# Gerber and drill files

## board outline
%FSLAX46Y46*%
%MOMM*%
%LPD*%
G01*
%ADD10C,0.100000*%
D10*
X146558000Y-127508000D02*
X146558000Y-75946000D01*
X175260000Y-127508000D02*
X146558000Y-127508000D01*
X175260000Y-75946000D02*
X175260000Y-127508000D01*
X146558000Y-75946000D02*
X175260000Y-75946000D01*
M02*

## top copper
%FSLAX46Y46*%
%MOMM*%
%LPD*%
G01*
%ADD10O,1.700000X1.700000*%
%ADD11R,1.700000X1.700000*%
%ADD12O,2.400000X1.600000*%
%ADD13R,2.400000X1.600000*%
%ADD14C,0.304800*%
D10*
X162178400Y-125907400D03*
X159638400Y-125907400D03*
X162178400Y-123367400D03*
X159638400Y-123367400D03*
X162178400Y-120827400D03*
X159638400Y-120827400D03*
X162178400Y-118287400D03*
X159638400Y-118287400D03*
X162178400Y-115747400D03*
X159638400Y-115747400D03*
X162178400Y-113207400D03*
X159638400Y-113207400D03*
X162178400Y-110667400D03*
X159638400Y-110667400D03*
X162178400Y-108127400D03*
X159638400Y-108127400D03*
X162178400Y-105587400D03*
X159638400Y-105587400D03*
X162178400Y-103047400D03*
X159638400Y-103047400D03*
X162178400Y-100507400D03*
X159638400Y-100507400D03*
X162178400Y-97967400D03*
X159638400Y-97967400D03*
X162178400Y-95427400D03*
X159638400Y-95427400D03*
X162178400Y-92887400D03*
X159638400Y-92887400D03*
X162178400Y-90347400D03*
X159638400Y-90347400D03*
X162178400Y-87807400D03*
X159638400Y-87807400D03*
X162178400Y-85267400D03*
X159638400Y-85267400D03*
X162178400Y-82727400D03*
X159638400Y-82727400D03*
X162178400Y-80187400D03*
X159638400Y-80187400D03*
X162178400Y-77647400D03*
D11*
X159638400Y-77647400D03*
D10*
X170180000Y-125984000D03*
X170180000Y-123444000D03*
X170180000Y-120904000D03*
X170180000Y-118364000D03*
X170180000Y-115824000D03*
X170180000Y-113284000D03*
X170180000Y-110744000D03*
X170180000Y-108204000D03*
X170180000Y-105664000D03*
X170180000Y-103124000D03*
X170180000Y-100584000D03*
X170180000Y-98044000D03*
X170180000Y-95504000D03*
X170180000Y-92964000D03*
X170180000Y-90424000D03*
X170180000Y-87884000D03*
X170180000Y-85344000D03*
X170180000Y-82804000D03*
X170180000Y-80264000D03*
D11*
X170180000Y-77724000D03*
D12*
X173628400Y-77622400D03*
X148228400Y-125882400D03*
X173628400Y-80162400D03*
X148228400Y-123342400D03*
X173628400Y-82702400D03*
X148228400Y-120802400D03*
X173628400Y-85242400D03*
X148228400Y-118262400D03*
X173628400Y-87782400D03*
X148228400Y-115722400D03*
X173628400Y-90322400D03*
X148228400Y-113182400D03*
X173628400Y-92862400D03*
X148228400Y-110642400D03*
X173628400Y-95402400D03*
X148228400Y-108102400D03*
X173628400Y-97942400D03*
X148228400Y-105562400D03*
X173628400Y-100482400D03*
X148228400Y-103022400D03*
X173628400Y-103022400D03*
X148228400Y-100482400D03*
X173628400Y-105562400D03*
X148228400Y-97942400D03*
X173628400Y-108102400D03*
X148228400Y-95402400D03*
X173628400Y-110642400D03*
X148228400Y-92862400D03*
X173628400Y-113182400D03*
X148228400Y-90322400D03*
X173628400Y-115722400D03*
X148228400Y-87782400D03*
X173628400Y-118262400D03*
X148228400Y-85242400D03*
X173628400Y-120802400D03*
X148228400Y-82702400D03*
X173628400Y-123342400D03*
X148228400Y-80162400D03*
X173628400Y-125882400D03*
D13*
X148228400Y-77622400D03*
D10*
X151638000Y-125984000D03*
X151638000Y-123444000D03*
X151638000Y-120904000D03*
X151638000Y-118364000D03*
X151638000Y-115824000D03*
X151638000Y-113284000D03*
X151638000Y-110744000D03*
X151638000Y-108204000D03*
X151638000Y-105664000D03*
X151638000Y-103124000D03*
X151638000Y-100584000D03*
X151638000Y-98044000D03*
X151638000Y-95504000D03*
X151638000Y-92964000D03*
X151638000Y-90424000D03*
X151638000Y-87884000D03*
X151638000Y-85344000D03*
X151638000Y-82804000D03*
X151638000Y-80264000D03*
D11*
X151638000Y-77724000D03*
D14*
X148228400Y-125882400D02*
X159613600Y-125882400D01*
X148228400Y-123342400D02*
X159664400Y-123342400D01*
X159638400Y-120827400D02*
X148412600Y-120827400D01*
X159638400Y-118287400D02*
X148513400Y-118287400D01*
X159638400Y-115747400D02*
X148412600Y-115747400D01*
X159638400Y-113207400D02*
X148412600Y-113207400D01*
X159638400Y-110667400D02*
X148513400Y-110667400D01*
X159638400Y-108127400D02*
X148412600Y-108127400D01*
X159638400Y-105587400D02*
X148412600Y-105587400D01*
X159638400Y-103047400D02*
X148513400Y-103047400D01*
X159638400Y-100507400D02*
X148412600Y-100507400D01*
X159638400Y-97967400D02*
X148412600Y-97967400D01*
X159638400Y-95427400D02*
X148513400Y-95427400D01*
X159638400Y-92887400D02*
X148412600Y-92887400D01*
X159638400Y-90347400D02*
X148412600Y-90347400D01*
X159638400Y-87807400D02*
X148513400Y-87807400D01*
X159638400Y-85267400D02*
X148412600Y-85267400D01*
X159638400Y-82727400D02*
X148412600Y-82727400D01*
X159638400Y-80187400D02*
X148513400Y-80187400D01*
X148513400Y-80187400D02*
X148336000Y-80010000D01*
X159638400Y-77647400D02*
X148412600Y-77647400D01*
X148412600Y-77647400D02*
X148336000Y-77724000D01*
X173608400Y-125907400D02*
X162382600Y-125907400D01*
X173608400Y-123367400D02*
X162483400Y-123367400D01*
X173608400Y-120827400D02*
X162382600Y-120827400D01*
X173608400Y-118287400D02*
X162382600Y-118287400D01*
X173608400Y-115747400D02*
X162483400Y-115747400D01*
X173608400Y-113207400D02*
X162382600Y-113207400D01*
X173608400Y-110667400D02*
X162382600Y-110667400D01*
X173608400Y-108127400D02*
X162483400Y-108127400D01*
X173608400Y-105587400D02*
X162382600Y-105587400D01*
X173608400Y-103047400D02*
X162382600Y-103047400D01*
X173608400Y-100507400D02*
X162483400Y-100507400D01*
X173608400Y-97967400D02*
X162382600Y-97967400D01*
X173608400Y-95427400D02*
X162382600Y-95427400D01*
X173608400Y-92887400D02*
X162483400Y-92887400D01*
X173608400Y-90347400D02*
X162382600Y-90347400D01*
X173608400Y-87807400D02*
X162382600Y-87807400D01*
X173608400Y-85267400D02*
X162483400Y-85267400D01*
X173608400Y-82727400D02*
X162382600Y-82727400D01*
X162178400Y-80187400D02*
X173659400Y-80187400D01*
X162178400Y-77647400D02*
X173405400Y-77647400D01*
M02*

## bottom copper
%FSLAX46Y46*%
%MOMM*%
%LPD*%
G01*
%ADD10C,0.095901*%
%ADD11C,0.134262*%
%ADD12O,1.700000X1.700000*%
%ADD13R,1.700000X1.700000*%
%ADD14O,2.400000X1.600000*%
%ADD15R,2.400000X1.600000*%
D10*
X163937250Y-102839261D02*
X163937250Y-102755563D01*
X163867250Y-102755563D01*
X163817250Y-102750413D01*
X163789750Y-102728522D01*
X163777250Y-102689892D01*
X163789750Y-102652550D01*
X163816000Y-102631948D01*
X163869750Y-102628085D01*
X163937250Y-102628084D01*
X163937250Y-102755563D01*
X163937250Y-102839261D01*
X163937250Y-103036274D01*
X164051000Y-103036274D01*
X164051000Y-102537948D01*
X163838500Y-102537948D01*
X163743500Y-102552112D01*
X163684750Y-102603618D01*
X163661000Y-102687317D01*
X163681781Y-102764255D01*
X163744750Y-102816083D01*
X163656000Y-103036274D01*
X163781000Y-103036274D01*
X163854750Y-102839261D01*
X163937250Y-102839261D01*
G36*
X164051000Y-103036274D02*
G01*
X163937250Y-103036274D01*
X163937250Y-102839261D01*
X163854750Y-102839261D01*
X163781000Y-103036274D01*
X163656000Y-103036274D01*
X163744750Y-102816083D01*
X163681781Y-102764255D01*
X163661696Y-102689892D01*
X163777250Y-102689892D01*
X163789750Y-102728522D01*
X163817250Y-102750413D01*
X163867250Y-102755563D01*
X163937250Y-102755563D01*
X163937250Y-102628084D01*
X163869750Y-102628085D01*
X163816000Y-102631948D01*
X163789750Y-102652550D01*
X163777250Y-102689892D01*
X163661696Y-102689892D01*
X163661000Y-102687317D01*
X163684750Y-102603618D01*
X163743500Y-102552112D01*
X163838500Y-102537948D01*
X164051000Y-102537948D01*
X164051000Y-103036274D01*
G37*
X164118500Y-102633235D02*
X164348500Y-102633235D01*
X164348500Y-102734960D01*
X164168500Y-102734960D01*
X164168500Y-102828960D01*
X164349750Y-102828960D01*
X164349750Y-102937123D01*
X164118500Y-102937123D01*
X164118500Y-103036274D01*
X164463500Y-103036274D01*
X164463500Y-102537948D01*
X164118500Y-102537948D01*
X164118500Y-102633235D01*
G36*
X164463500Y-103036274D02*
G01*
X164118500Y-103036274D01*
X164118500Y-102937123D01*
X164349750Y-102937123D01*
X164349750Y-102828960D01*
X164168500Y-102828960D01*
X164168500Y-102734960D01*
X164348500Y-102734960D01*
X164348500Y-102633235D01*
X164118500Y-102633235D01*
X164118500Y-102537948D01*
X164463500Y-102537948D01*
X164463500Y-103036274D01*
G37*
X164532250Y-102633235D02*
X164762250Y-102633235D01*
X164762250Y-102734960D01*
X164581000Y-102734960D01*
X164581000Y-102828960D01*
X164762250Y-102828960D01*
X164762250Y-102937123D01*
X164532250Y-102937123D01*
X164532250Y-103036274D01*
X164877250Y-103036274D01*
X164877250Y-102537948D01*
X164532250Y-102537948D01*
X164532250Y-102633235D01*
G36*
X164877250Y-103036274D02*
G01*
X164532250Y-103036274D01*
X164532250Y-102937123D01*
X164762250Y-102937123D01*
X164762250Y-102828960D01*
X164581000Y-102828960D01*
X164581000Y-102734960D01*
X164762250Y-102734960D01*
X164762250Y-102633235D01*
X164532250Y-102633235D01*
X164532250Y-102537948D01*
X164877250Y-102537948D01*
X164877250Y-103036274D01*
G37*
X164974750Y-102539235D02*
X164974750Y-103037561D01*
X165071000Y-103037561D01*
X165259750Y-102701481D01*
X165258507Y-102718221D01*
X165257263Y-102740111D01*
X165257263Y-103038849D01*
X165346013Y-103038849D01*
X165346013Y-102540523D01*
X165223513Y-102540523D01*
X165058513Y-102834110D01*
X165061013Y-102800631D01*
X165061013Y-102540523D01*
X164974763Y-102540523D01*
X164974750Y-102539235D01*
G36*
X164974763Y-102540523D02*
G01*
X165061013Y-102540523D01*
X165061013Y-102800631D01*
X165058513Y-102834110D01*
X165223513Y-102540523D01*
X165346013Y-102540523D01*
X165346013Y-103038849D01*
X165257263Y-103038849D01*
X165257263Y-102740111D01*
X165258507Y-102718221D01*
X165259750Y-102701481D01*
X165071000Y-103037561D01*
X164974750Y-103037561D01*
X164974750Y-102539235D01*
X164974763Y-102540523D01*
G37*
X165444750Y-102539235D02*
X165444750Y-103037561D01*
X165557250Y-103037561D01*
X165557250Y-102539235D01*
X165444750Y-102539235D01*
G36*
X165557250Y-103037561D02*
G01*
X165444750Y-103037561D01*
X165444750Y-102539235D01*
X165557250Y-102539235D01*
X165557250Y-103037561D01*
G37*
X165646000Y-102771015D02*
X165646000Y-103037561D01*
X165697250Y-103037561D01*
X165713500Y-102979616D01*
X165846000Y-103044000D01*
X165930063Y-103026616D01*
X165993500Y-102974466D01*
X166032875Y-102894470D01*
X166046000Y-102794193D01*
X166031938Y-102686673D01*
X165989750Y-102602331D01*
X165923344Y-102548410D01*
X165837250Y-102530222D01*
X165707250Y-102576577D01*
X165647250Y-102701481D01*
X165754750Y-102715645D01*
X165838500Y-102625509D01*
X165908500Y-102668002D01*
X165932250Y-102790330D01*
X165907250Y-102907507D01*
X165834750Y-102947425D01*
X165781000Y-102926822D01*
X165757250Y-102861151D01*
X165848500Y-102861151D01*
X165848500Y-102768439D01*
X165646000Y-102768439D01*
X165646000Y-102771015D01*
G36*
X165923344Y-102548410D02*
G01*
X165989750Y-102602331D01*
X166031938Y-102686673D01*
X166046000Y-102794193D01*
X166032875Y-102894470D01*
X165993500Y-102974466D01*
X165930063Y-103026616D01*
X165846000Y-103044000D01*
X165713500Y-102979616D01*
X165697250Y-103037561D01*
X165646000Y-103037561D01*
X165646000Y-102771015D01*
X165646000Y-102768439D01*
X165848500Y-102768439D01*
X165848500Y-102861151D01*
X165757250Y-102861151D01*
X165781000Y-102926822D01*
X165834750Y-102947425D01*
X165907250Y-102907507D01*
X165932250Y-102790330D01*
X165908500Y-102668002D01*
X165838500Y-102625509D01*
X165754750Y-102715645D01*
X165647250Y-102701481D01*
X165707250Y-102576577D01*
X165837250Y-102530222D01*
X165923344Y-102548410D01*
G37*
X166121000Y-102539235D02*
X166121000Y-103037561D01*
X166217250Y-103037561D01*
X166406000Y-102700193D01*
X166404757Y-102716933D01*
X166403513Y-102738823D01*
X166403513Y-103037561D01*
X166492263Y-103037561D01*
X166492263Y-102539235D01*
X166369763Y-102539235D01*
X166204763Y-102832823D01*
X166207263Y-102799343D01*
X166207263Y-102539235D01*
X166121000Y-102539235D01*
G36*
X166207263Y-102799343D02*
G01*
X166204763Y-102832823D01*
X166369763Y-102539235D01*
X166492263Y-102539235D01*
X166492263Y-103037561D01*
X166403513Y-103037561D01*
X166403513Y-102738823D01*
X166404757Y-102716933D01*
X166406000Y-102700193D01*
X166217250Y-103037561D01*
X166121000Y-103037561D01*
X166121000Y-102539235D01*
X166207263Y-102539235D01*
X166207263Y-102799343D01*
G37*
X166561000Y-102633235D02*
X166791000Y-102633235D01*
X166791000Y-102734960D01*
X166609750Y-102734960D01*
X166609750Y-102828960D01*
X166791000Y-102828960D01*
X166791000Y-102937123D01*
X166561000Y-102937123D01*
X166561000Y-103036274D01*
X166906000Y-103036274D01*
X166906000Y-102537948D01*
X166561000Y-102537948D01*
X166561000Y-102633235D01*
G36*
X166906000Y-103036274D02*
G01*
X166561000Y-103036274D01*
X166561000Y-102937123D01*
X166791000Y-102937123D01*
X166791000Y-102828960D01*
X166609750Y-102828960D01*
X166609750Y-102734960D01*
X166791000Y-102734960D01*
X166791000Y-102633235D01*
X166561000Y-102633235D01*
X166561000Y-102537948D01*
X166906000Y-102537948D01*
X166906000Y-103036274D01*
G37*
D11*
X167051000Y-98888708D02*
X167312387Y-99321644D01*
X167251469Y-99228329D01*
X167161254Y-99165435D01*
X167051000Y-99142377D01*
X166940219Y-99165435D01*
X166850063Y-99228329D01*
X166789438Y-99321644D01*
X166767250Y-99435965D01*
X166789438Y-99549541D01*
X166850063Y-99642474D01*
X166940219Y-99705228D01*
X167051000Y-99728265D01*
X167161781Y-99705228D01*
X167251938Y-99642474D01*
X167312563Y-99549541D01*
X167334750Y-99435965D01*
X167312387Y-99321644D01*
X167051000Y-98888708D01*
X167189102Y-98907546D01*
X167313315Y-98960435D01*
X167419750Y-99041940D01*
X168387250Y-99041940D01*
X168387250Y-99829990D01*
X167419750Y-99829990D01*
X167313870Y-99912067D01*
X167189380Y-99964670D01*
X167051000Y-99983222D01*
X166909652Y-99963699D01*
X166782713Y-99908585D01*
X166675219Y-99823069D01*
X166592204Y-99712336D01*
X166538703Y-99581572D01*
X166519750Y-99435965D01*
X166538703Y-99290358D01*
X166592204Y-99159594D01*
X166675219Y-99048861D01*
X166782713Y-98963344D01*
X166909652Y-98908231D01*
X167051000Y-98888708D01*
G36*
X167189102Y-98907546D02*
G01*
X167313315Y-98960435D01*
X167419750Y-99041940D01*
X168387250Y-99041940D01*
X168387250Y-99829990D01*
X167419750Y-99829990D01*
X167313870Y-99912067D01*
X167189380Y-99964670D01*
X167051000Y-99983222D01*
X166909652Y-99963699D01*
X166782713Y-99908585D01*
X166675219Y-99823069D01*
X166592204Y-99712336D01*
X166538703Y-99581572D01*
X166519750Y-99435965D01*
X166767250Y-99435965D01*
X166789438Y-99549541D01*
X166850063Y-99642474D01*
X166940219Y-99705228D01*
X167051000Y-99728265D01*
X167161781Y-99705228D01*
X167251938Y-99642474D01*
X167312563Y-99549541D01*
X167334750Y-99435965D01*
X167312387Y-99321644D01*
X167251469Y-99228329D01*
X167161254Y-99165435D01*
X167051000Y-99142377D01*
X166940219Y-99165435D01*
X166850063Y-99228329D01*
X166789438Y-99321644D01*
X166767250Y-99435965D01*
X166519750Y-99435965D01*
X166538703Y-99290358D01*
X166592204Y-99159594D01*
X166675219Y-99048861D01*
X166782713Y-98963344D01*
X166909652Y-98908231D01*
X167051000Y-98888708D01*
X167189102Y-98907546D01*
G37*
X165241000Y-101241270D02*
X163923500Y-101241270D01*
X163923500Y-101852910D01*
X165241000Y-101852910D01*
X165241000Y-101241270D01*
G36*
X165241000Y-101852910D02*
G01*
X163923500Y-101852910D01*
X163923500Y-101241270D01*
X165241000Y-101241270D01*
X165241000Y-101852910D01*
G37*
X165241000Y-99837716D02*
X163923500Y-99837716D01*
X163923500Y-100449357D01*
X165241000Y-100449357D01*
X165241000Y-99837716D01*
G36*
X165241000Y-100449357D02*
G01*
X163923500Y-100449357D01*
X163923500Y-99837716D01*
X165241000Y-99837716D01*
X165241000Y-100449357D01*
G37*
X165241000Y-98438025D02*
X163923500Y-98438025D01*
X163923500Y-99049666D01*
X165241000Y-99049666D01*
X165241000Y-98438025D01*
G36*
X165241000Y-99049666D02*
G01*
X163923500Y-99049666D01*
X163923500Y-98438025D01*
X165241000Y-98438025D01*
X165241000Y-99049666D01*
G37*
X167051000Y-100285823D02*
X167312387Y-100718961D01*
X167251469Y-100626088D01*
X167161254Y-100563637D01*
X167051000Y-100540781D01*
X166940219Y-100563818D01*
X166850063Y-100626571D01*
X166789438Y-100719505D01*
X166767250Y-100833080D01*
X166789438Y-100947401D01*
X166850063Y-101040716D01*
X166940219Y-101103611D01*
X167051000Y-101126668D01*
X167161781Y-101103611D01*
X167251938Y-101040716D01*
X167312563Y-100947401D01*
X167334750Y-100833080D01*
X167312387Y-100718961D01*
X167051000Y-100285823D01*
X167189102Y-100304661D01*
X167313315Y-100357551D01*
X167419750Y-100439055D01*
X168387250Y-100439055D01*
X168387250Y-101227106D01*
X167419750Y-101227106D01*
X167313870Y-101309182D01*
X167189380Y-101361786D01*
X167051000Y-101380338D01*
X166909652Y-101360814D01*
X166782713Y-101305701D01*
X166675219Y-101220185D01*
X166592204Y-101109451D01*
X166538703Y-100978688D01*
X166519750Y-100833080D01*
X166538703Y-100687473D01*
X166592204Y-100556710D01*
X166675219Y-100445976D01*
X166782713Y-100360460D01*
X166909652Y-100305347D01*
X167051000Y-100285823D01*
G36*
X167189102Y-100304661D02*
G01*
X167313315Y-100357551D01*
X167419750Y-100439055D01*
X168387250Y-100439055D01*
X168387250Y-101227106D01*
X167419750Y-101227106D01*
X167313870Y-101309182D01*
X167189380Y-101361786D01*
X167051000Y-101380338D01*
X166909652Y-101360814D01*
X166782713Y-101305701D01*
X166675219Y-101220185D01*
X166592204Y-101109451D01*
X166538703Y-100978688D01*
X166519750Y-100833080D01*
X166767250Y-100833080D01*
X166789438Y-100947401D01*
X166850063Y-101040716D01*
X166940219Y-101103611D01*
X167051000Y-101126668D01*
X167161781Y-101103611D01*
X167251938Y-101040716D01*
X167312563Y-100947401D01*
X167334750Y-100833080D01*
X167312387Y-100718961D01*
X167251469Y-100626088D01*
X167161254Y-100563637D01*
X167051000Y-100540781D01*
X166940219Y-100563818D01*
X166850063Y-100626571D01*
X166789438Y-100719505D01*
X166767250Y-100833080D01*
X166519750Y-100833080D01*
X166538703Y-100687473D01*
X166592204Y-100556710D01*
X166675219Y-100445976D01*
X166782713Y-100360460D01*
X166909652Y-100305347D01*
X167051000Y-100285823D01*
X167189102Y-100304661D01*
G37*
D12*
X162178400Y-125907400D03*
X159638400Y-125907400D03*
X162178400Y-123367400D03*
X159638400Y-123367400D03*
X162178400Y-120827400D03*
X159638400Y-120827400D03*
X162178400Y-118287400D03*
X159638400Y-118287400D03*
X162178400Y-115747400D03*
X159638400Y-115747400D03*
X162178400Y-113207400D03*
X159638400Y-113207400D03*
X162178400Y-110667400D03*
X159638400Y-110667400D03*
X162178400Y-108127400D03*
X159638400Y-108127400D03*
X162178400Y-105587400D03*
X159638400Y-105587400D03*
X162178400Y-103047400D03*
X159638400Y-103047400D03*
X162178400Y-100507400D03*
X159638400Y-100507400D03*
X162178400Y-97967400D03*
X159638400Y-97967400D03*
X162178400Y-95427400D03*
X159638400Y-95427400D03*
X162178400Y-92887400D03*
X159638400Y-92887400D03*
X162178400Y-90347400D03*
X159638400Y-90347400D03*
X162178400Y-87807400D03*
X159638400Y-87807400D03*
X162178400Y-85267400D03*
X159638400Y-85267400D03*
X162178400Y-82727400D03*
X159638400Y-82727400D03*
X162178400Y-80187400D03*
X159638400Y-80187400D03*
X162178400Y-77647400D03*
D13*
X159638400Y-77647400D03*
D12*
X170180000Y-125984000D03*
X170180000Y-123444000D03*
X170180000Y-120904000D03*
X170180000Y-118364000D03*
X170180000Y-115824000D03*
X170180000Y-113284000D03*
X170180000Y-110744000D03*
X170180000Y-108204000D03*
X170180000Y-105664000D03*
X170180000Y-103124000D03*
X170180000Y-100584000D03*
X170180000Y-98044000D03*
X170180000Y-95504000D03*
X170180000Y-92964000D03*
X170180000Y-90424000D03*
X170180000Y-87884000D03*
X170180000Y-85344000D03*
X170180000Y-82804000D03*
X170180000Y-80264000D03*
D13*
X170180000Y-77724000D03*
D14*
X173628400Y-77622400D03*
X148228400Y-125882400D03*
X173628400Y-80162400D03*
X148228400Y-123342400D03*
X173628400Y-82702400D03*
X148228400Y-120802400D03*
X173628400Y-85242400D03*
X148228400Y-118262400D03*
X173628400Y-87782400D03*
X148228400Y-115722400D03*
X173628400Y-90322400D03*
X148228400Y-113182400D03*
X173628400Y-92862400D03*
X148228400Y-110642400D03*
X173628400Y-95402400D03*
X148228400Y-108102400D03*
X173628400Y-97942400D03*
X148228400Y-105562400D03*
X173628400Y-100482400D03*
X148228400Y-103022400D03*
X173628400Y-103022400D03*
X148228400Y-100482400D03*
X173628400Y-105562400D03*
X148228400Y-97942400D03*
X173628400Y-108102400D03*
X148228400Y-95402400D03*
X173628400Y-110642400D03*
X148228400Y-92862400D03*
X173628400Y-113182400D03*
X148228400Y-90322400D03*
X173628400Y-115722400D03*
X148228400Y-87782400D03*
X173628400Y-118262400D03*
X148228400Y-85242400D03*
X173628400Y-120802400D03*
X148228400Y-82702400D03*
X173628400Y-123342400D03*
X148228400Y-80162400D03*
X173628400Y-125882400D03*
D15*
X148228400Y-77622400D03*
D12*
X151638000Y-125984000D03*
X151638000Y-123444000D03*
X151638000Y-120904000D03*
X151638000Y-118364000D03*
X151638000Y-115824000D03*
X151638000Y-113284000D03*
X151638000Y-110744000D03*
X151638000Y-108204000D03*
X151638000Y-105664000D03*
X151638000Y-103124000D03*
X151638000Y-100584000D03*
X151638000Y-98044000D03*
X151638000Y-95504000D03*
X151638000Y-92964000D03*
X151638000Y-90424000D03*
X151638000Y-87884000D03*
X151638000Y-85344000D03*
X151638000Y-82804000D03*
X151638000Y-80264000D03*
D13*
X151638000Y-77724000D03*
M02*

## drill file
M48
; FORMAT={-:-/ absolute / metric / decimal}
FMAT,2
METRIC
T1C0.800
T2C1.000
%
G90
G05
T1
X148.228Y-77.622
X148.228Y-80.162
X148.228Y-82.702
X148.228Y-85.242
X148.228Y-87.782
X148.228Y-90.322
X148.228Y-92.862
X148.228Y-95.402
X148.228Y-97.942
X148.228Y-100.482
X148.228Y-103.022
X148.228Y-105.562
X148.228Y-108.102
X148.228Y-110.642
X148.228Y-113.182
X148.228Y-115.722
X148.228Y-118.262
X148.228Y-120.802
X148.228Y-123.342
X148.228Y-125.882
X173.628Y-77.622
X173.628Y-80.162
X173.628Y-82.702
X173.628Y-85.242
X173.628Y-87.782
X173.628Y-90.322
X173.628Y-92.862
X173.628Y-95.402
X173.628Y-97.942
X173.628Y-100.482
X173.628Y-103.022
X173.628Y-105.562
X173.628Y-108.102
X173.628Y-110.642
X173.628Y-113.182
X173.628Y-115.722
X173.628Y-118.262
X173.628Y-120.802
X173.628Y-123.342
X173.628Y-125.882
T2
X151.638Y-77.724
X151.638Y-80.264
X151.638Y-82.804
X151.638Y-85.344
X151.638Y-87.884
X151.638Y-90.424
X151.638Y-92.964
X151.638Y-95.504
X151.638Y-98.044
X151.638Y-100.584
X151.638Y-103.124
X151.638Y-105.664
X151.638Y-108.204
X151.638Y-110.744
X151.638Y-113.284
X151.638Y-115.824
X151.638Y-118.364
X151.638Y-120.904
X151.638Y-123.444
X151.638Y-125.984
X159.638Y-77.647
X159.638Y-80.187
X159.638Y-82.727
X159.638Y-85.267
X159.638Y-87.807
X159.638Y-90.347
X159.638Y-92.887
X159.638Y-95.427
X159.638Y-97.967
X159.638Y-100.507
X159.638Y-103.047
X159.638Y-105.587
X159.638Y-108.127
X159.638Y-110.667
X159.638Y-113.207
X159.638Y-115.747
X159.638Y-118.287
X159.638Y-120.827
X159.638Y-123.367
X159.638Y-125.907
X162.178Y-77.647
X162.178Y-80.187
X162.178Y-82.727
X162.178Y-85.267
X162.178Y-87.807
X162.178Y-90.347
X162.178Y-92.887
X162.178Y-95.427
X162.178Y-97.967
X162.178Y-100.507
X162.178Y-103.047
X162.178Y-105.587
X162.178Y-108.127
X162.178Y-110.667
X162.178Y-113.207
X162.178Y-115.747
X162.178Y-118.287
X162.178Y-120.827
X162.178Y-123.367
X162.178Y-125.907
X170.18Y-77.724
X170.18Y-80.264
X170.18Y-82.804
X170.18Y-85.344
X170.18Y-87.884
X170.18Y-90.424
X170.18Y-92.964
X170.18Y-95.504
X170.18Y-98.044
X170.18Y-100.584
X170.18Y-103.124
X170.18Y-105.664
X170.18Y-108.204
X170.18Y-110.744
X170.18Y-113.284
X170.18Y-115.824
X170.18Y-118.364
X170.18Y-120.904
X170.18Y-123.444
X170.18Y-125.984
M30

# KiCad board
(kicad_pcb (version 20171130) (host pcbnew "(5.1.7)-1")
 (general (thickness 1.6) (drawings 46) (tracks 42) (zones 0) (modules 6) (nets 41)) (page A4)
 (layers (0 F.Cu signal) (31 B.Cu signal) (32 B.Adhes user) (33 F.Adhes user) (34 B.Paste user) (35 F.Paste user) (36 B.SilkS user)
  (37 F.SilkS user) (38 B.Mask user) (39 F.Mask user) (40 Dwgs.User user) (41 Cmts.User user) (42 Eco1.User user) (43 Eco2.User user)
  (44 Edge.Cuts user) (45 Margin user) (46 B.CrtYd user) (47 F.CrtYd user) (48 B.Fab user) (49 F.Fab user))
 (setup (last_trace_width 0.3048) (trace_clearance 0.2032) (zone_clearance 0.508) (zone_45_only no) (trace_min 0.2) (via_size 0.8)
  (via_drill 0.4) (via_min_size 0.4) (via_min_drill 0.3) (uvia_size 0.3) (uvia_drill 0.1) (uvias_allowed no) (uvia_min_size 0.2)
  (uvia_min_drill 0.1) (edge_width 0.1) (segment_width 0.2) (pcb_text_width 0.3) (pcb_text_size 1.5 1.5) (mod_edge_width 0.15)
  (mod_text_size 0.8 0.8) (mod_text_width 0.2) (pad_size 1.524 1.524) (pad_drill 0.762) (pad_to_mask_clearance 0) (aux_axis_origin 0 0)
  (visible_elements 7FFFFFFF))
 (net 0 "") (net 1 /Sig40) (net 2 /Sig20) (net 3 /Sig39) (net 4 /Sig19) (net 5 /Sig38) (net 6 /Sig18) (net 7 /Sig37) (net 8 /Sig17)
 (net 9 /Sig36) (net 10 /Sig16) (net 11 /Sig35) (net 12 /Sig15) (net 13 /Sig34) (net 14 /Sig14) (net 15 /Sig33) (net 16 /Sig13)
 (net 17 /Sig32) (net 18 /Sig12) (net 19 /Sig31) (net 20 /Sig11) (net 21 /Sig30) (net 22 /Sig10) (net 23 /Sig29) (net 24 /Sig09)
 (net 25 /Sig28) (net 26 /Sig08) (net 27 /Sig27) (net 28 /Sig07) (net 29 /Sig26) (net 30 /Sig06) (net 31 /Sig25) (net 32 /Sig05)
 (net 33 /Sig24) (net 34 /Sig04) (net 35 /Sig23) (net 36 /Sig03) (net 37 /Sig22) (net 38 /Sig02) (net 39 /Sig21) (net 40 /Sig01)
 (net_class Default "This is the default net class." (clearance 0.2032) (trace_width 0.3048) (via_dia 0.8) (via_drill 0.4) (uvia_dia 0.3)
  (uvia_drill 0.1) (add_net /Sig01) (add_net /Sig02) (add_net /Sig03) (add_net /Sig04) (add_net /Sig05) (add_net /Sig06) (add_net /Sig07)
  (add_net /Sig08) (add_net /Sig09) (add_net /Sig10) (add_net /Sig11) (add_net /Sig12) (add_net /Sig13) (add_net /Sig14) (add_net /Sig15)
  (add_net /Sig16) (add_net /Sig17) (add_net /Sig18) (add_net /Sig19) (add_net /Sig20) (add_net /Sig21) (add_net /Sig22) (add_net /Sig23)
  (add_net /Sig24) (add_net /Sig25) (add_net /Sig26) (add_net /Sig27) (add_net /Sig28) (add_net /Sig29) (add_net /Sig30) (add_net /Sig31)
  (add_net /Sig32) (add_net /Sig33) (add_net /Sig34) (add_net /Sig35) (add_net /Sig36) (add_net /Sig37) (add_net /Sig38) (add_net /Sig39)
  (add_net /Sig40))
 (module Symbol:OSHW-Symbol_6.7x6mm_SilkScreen (layer F.Cu) (at 166.116 100.584 90)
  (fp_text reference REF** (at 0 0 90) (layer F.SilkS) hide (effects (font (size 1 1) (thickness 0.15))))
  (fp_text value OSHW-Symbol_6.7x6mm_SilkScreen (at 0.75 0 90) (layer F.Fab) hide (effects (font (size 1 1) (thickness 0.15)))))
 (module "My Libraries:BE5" (layer B.Cu) (at 168.656 98.044 180)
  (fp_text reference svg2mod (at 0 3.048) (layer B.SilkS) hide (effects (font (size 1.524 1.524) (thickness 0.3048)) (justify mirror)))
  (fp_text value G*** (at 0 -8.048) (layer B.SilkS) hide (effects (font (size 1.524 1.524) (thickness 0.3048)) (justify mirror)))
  (fp_poly
   (pts (xy 4.71875 -4.795261) (xy 4.71875 -4.711563) (xy 4.78875 -4.711563) (xy 4.83875 -4.706413) (xy 4.86625 -4.684522)
    (xy 4.87875 -4.645892) (xy 4.86625 -4.60855) (xy 4.84 -4.587948) (xy 4.78625 -4.584085) (xy 4.71875 -4.584084) (xy 4.71875 -4.711563)
    (xy 4.71875 -4.795261) (xy 4.71875 -4.992274) (xy 4.605 -4.992274) (xy 4.605 -4.493948) (xy 4.8175 -4.493948) (xy 4.9125 -4.508112)
    (xy 4.97125 -4.559618) (xy 4.995 -4.643317) (xy 4.974219 -4.720255) (xy 4.91125 -4.772083) (xy 5 -4.992274) (xy 4.875 -4.992274)
    (xy 4.80125 -4.795261) (xy 4.71875 -4.795261))
   (layer B.Cu) (width 0.095901))
  (fp_poly
   (pts (xy 4.5375 -4.589235) (xy 4.3075 -4.589235) (xy 4.3075 -4.69096) (xy 4.4875 -4.69096) (xy 4.4875 -4.78496) (xy 4.30625 -4.78496)
    (xy 4.30625 -4.893123) (xy 4.5375 -4.893123) (xy 4.5375 -4.992274) (xy 4.1925 -4.992274) (xy 4.1925 -4.493948) (xy 4.5375 -4.493948)
    (xy 4.5375 -4.589235))
   (layer B.Cu) (width 0.095901))
  (fp_poly
   (pts (xy 4.12375 -4.589235) (xy 3.89375 -4.589235) (xy 3.89375 -4.69096) (xy 4.075 -4.69096) (xy 4.075 -4.78496) (xy 3.89375 -4.78496)
    (xy 3.89375 -4.893123) (xy 4.12375 -4.893123) (xy 4.12375 -4.992274) (xy 3.77875 -4.992274) (xy 3.77875 -4.493948)
    (xy 4.12375 -4.493948) (xy 4.12375 -4.589235))
   (layer B.Cu) (width 0.095901))
  (fp_poly
   (pts (xy 3.68125 -4.495235) (xy 3.68125 -4.993561) (xy 3.585 -4.993561) (xy 3.39625 -4.657481) (xy 3.397493 -4.674221)
    (xy 3.398737 -4.696111) (xy 3.398737 -4.994849) (xy 3.309987 -4.994849) (xy 3.309987 -4.496523) (xy 3.432487 -4.496523)
    (xy 3.597487 -4.79011) (xy 3.594987 -4.756631) (xy 3.594987 -4.496523) (xy 3.681237 -4.496523) (xy 3.68125 -4.495235))
   (layer B.Cu) (width 0.095901))
  (fp_poly
   (pts (xy 3.21125 -4.495235) (xy 3.21125 -4.993561) (xy 3.09875 -4.993561) (xy 3.09875 -4.495235) (xy 3.21125 -4.495235)) (layer B.Cu)
   (width 0.095901))
  (fp_poly
   (pts (xy 3.01 -4.727015) (xy 3.01 -4.993561) (xy 2.95875 -4.993561) (xy 2.9425 -4.935616) (xy 2.81 -5) (xy 2.725937 -4.982616)
    (xy 2.6625 -4.930466) (xy 2.623125 -4.85047) (xy 2.61 -4.750193) (xy 2.624062 -4.642673) (xy 2.66625 -4.558331) (xy 2.732656 -4.50441)
    (xy 2.81875 -4.486222) (xy 2.94875 -4.532577) (xy 3.00875 -4.657481) (xy 2.90125 -4.671645) (xy 2.8175 -4.581509) (xy 2.7475 -4.624002)
    (xy 2.72375 -4.74633) (xy 2.74875 -4.863507) (xy 2.82125 -4.903425) (xy 2.875 -4.882822) (xy 2.89875 -4.817151) (xy 2.8075 -4.817151)
    (xy 2.8075 -4.724439) (xy 3.01 -4.724439) (xy 3.01 -4.727015))
   (layer B.Cu) (width 0.095901))
  (fp_poly
   (pts (xy 2.535 -4.495235) (xy 2.535 -4.993561) (xy 2.43875 -4.993561) (xy 2.25 -4.656193) (xy 2.251243 -4.672933) (xy 2.252487 -4.694823)
    (xy 2.252487 -4.993561) (xy 2.163737 -4.993561) (xy 2.163737 -4.495235) (xy 2.286237 -4.495235) (xy 2.451237 -4.788823)
    (xy 2.448737 -4.755343) (xy 2.448737 -4.495235) (xy 2.535 -4.495235))
   (layer B.Cu) (width 0.095901))
  (fp_poly
   (pts (xy 2.095 -4.589235) (xy 1.865 -4.589235) (xy 1.865 -4.69096) (xy 2.04625 -4.69096) (xy 2.04625 -4.78496) (xy 1.865 -4.78496)
    (xy 1.865 -4.893123) (xy 2.095 -4.893123) (xy 2.095 -4.992274) (xy 1.75 -4.992274) (xy 1.75 -4.493948) (xy 2.095 -4.493948)
    (xy 2.095 -4.589235))
   (layer B.Cu) (width 0.095901))
  (fp_poly
   (pts (xy 1.605 -0.844708) (xy 1.343613 -1.277644) (xy 1.404531 -1.184329) (xy 1.494746 -1.121435) (xy 1.605 -1.098377)
    (xy 1.715781 -1.121435) (xy 1.805937 -1.184329) (xy 1.866562 -1.277644) (xy 1.88875 -1.391965) (xy 1.866562 -1.505541)
    (xy 1.805937 -1.598474) (xy 1.715781 -1.661228) (xy 1.605 -1.684265) (xy 1.494219 -1.661228) (xy 1.404062 -1.598474)
    (xy 1.343437 -1.505541) (xy 1.32125 -1.391965) (xy 1.343613 -1.277644) (xy 1.605 -0.844708) (xy 1.466898 -0.863546)
    (xy 1.342685 -0.916435) (xy 1.23625 -0.99794) (xy 0.26875 -0.99794) (xy 0.26875 -1.78599) (xy 1.23625 -1.78599) (xy 1.34213 -1.868067)
    (xy 1.46662 -1.92067) (xy 1.605 -1.939222) (xy 1.746348 -1.919699) (xy 1.873287 -1.864585) (xy 1.980781 -1.779069)
    (xy 2.063796 -1.668336) (xy 2.117297 -1.537572) (xy 2.13625 -1.391965) (xy 2.117297 -1.246358) (xy 2.063796 -1.115594)
    (xy 1.980781 -1.004861) (xy 1.873287 -0.919344) (xy 1.746348 -0.864231) (xy 1.605 -0.844708))
   (layer B.Cu) (width 0.134262))
  (fp_poly
   (pts (xy 3.415 -3.19727) (xy 4.7325 -3.19727) (xy 4.7325 -3.80891) (xy 3.415 -3.80891) (xy 3.415 -3.19727)) (layer B.Cu) (width 0.134262))
  (fp_poly
   (pts (xy 3.415 -1.793716) (xy 4.7325 -1.793716) (xy 4.7325 -2.405357) (xy 3.415 -2.405357) (xy 3.415 -1.793716)) (layer B.Cu)
   (width 0.134262))
  (fp_poly
   (pts (xy 3.415 -0.394025) (xy 4.7325 -0.394025) (xy 4.7325 -1.005666) (xy 3.415 -1.005666) (xy 3.415 -0.394025)) (layer B.Cu)
   (width 0.134262))
  (fp_poly
   (pts (xy 1.605 -2.241823) (xy 1.343613 -2.674961) (xy 1.404531 -2.582088) (xy 1.494746 -2.519637) (xy 1.605 -2.496781)
    (xy 1.715781 -2.519818) (xy 1.805937 -2.582571) (xy 1.866562 -2.675505) (xy 1.88875 -2.78908) (xy 1.866562 -2.903401)
    (xy 1.805937 -2.996716) (xy 1.715781 -3.059611) (xy 1.605 -3.082668) (xy 1.494219 -3.059611) (xy 1.404062 -2.996716)
    (xy 1.343437 -2.903401) (xy 1.32125 -2.78908) (xy 1.343613 -2.674961) (xy 1.605 -2.241823) (xy 1.466898 -2.260661)
    (xy 1.342685 -2.313551) (xy 1.23625 -2.395055) (xy 0.26875 -2.395055) (xy 0.26875 -3.183106) (xy 1.23625 -3.183106)
    (xy 1.34213 -3.265182) (xy 1.46662 -3.317786) (xy 1.605 -3.336338) (xy 1.746348 -3.316814) (xy 1.873287 -3.261701)
    (xy 1.980781 -3.176185) (xy 2.063796 -3.065451) (xy 2.117297 -2.934688) (xy 2.13625 -2.78908) (xy 2.117297 -2.643473)
    (xy 2.063796 -2.51271) (xy 1.980781 -2.401976) (xy 1.873287 -2.31646) (xy 1.746348 -2.261347) (xy 1.605 -2.241823))
   (layer B.Cu) (width 0.134262)))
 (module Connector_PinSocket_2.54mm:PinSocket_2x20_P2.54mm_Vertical (layer B.Cu) (at 159.6384 77.6474 180)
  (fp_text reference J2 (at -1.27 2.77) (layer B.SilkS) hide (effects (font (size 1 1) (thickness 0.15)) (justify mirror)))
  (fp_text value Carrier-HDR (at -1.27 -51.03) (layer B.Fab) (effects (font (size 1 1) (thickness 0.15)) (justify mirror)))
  (pad 40 thru_hole oval (at -2.54 -48.26 180) (size 1.7 1.7) (drill 1) (layers *.Cu *.Mask) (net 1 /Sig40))
  (pad 39 thru_hole oval (at 0 -48.26 180) (size 1.7 1.7) (drill 1) (layers *.Cu *.Mask) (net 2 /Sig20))
  (pad 38 thru_hole oval (at -2.54 -45.72 180) (size 1.7 1.7) (drill 1) (layers *.Cu *.Mask) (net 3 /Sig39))
  (pad 37 thru_hole oval (at 0 -45.72 180) (size 1.7 1.7) (drill 1) (layers *.Cu *.Mask) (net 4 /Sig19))
  (pad 36 thru_hole oval (at -2.54 -43.18 180) (size 1.7 1.7) (drill 1) (layers *.Cu *.Mask) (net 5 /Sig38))
  (pad 35 thru_hole oval (at 0 -43.18 180) (size 1.7 1.7) (drill 1) (layers *.Cu *.Mask) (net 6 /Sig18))
  (pad 34 thru_hole oval (at -2.54 -40.64 180) (size 1.7 1.7) (drill 1) (layers *.Cu *.Mask) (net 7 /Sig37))
  (pad 33 thru_hole oval (at 0 -40.64 180) (size 1.7 1.7) (drill 1) (layers *.Cu *.Mask) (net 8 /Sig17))
  (pad 32 thru_hole oval (at -2.54 -38.1 180) (size 1.7 1.7) (drill 1) (layers *.Cu *.Mask) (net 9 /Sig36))
  (pad 31 thru_hole oval (at 0 -38.1 180) (size 1.7 1.7) (drill 1) (layers *.Cu *.Mask) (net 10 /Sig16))
  (pad 30 thru_hole oval (at -2.54 -35.56 180) (size 1.7 1.7) (drill 1) (layers *.Cu *.Mask) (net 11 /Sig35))
  (pad 29 thru_hole oval (at 0 -35.56 180) (size 1.7 1.7) (drill 1) (layers *.Cu *.Mask) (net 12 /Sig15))
  (pad 28 thru_hole oval (at -2.54 -33.02 180) (size 1.7 1.7) (drill 1) (layers *.Cu *.Mask) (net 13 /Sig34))
  (pad 27 thru_hole oval (at 0 -33.02 180) (size 1.7 1.7) (drill 1) (layers *.Cu *.Mask) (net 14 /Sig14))
  (pad 26 thru_hole oval (at -2.54 -30.48 180) (size 1.7 1.7) (drill 1) (layers *.Cu *.Mask) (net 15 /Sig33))
  (pad 25 thru_hole oval (at 0 -30.48 180) (size 1.7 1.7) (drill 1) (layers *.Cu *.Mask) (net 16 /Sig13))
  (pad 24 thru_hole oval (at -2.54 -27.94 180) (size 1.7 1.7) (drill 1) (layers *.Cu *.Mask) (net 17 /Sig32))
  (pad 23 thru_hole oval (at 0 -27.94 180) (size 1.7 1.7) (drill 1) (layers *.Cu *.Mask) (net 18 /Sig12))
  (pad 22 thru_hole oval (at -2.54 -25.4 180) (size 1.7 1.7) (drill 1) (layers *.Cu *.Mask) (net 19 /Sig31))
  (pad 21 thru_hole oval (at 0 -25.4 180) (size 1.7 1.7) (drill 1) (layers *.Cu *.Mask) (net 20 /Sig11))
  (pad 20 thru_hole oval (at -2.54 -22.86 180) (size 1.7 1.7) (drill 1) (layers *.Cu *.Mask) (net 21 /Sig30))
  (pad 19 thru_hole oval (at 0 -22.86 180) (size 1.7 1.7) (drill 1) (layers *.Cu *.Mask) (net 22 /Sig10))
  (pad 18 thru_hole oval (at -2.54 -20.32 180) (size 1.7 1.7) (drill 1) (layers *.Cu *.Mask) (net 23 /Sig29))
  (pad 17 thru_hole oval (at 0 -20.32 180) (size 1.7 1.7) (drill 1) (layers *.Cu *.Mask) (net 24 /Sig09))
  (pad 16 thru_hole oval (at -2.54 -17.78 180) (size 1.7 1.7) (drill 1) (layers *.Cu *.Mask) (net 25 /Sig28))
  (pad 15 thru_hole oval (at 0 -17.78 180) (size 1.7 1.7) (drill 1) (layers *.Cu *.Mask) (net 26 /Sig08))
  (pad 14 thru_hole oval (at -2.54 -15.24 180) (size 1.7 1.7) (drill 1) (layers *.Cu *.Mask) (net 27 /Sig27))
  (pad 13 thru_hole oval (at 0 -15.24 180) (size 1.7 1.7) (drill 1) (layers *.Cu *.Mask) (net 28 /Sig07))
  (pad 12 thru_hole oval (at -2.54 -12.7 180) (size 1.7 1.7) (drill 1) (layers *.Cu *.Mask) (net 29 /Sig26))
  (pad 11 thru_hole oval (at 0 -12.7 180) (size 1.7 1.7) (drill 1) (layers *.Cu *.Mask) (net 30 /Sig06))
  (pad 10 thru_hole oval (at -2.54 -10.16 180) (size 1.7 1.7) (drill 1) (layers *.Cu *.Mask) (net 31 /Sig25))
  (pad 9 thru_hole oval (at 0 -10.16 180) (size 1.7 1.7) (drill 1) (layers *.Cu *.Mask) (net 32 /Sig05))
  (pad 8 thru_hole oval (at -2.54 -7.62 180) (size 1.7 1.7) (drill 1) (layers *.Cu *.Mask) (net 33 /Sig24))
  (pad 7 thru_hole oval (at 0 -7.62 180) (size 1.7 1.7) (drill 1) (layers *.Cu *.Mask) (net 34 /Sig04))
  (pad 6 thru_hole oval (at -2.54 -5.08 180) (size 1.7 1.7) (drill 1) (layers *.Cu *.Mask) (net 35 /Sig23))
  (pad 5 thru_hole oval (at 0 -5.08 180) (size 1.7 1.7) (drill 1) (layers *.Cu *.Mask) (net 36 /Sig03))
  (pad 4 thru_hole oval (at -2.54 -2.54 180) (size 1.7 1.7) (drill 1) (layers *.Cu *.Mask) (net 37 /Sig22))
  (pad 3 thru_hole oval (at 0 -2.54 180) (size 1.7 1.7) (drill 1) (layers *.Cu *.Mask) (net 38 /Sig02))
  (pad 2 thru_hole oval (at -2.54 0 180) (size 1.7 1.7) (drill 1) (layers *.Cu *.Mask) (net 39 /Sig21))
  (pad 1 thru_hole rect (at 0 0 180) (size 1.7 1.7) (drill 1) (layers *.Cu *.Mask) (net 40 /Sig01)))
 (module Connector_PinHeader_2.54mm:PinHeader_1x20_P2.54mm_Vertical (layer F.Cu) (at 170.18 77.724)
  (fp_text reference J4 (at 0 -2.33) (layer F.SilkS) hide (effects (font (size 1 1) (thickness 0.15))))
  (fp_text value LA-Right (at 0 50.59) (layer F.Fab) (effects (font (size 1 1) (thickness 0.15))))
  (pad 20 thru_hole oval (at 0 48.26) (size 1.7 1.7) (drill 1) (layers *.Cu *.Mask) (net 1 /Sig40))
  (pad 19 thru_hole oval (at 0 45.72) (size 1.7 1.7) (drill 1) (layers *.Cu *.Mask) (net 3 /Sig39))
  (pad 18 thru_hole oval (at 0 43.18) (size 1.7 1.7) (drill 1) (layers *.Cu *.Mask) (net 5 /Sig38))
  (pad 17 thru_hole oval (at 0 40.64) (size 1.7 1.7) (drill 1) (layers *.Cu *.Mask) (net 7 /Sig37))
  (pad 16 thru_hole oval (at 0 38.1) (size 1.7 1.7) (drill 1) (layers *.Cu *.Mask) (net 9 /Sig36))
  (pad 15 thru_hole oval (at 0 35.56) (size 1.7 1.7) (drill 1) (layers *.Cu *.Mask) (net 11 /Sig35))
  (pad 14 thru_hole oval (at 0 33.02) (size 1.7 1.7) (drill 1) (layers *.Cu *.Mask) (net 13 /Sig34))
  (pad 13 thru_hole oval (at 0 30.48) (size 1.7 1.7) (drill 1) (layers *.Cu *.Mask) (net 15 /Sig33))
  (pad 12 thru_hole oval (at 0 27.94) (size 1.7 1.7) (drill 1) (layers *.Cu *.Mask) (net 17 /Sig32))
  (pad 11 thru_hole oval (at 0 25.4) (size 1.7 1.7) (drill 1) (layers *.Cu *.Mask) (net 19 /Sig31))
  (pad 10 thru_hole oval (at 0 22.86) (size 1.7 1.7) (drill 1) (layers *.Cu *.Mask) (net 21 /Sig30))
  (pad 9 thru_hole oval (at 0 20.32) (size 1.7 1.7) (drill 1) (layers *.Cu *.Mask) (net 23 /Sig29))
  (pad 8 thru_hole oval (at 0 17.78) (size 1.7 1.7) (drill 1) (layers *.Cu *.Mask) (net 25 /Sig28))
  (pad 7 thru_hole oval (at 0 15.24) (size 1.7 1.7) (drill 1) (layers *.Cu *.Mask) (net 27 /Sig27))
  (pad 6 thru_hole oval (at 0 12.7) (size 1.7 1.7) (drill 1) (layers *.Cu *.Mask) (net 29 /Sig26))
  (pad 5 thru_hole oval (at 0 10.16) (size 1.7 1.7) (drill 1) (layers *.Cu *.Mask) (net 31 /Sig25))
  (pad 4 thru_hole oval (at 0 7.62) (size 1.7 1.7) (drill 1) (layers *.Cu *.Mask) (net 33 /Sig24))
  (pad 3 thru_hole oval (at 0 5.08) (size 1.7 1.7) (drill 1) (layers *.Cu *.Mask) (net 35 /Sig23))
  (pad 2 thru_hole oval (at 0 2.54) (size 1.7 1.7) (drill 1) (layers *.Cu *.Mask) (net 37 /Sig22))
  (pad 1 thru_hole rect (at 0 0) (size 1.7 1.7) (drill 1) (layers *.Cu *.Mask) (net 39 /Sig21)))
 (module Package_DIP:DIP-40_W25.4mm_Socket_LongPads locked (layer F.Cu) (at 148.2284 77.6224)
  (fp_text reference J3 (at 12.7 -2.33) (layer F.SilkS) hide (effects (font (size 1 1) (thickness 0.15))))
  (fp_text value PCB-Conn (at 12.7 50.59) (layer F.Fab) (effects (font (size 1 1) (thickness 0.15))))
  (pad 40 thru_hole oval (at 25.4 0) (size 2.4 1.6) (drill 0.8) (layers *.Cu *.Mask) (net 39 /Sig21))
  (pad 20 thru_hole oval (at 0 48.26) (size 2.4 1.6) (drill 0.8) (layers *.Cu *.Mask) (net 2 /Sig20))
  (pad 39 thru_hole oval (at 25.4 2.54) (size 2.4 1.6) (drill 0.8) (layers *.Cu *.Mask) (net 37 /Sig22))
  (pad 19 thru_hole oval (at 0 45.72) (size 2.4 1.6) (drill 0.8) (layers *.Cu *.Mask) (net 4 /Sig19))
  (pad 38 thru_hole oval (at 25.4 5.08) (size 2.4 1.6) (drill 0.8) (layers *.Cu *.Mask) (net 35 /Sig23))
  (pad 18 thru_hole oval (at 0 43.18) (size 2.4 1.6) (drill 0.8) (layers *.Cu *.Mask) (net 6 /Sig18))
  (pad 37 thru_hole oval (at 25.4 7.62) (size 2.4 1.6) (drill 0.8) (layers *.Cu *.Mask) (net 33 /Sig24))
  (pad 17 thru_hole oval (at 0 40.64) (size 2.4 1.6) (drill 0.8) (layers *.Cu *.Mask) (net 8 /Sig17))
  (pad 36 thru_hole oval (at 25.4 10.16) (size 2.4 1.6) (drill 0.8) (layers *.Cu *.Mask) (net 31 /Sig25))
  (pad 16 thru_hole oval (at 0 38.1) (size 2.4 1.6) (drill 0.8) (layers *.Cu *.Mask) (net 10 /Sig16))
  (pad 35 thru_hole oval (at 25.4 12.7) (size 2.4 1.6) (drill 0.8) (layers *.Cu *.Mask) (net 29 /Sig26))
  (pad 15 thru_hole oval (at 0 35.56) (size 2.4 1.6) (drill 0.8) (layers *.Cu *.Mask) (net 12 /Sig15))
  (pad 34 thru_hole oval (at 25.4 15.24) (size 2.4 1.6) (drill 0.8) (layers *.Cu *.Mask) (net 27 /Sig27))
  (pad 14 thru_hole oval (at 0 33.02) (size 2.4 1.6) (drill 0.8) (layers *.Cu *.Mask) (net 14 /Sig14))
  (pad 33 thru_hole oval (at 25.4 17.78) (size 2.4 1.6) (drill 0.8) (layers *.Cu *.Mask) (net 25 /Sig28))
  (pad 13 thru_hole oval (at 0 30.48) (size 2.4 1.6) (drill 0.8) (layers *.Cu *.Mask) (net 16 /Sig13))
  (pad 32 thru_hole oval (at 25.4 20.32) (size 2.4 1.6) (drill 0.8) (layers *.Cu *.Mask) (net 23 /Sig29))
  (pad 12 thru_hole oval (at 0 27.94) (size 2.4 1.6) (drill 0.8) (layers *.Cu *.Mask) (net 18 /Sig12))
  (pad 31 thru_hole oval (at 25.4 22.86) (size 2.4 1.6) (drill 0.8) (layers *.Cu *.Mask) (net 21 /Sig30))
  (pad 11 thru_hole oval (at 0 25.4) (size 2.4 1.6) (drill 0.8) (layers *.Cu *.Mask) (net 20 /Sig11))
  (pad 30 thru_hole oval (at 25.4 25.4) (size 2.4 1.6) (drill 0.8) (layers *.Cu *.Mask) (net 19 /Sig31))
  (pad 10 thru_hole oval (at 0 22.86) (size 2.4 1.6) (drill 0.8) (layers *.Cu *.Mask) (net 22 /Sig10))
  (pad 29 thru_hole oval (at 25.4 27.94) (size 2.4 1.6) (drill 0.8) (layers *.Cu *.Mask) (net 17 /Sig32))
  (pad 9 thru_hole oval (at 0 20.32) (size 2.4 1.6) (drill 0.8) (layers *.Cu *.Mask) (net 24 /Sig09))
  (pad 28 thru_hole oval (at 25.4 30.48) (size 2.4 1.6) (drill 0.8) (layers *.Cu *.Mask) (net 15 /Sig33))
  (pad 8 thru_hole oval (at 0 17.78) (size 2.4 1.6) (drill 0.8) (layers *.Cu *.Mask) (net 26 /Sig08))
  (pad 27 thru_hole oval (at 25.4 33.02) (size 2.4 1.6) (drill 0.8) (layers *.Cu *.Mask) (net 13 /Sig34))
  (pad 7 thru_hole oval (at 0 15.24) (size 2.4 1.6) (drill 0.8) (layers *.Cu *.Mask) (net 28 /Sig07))
  (pad 26 thru_hole oval (at 25.4 35.56) (size 2.4 1.6) (drill 0.8) (layers *.Cu *.Mask) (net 11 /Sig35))
  (pad 6 thru_hole oval (at 0 12.7) (size 2.4 1.6) (drill 0.8) (layers *.Cu *.Mask) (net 30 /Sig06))
  (pad 25 thru_hole oval (at 25.4 38.1) (size 2.4 1.6) (drill 0.8) (layers *.Cu *.Mask) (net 9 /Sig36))
  (pad 5 thru_hole oval (at 0 10.16) (size 2.4 1.6) (drill 0.8) (layers *.Cu *.Mask) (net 32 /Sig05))
  (pad 24 thru_hole oval (at 25.4 40.64) (size 2.4 1.6) (drill 0.8) (layers *.Cu *.Mask) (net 7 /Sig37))
  (pad 4 thru_hole oval (at 0 7.62) (size 2.4 1.6) (drill 0.8) (layers *.Cu *.Mask) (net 34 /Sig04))
  (pad 23 thru_hole oval (at 25.4 43.18) (size 2.4 1.6) (drill 0.8) (layers *.Cu *.Mask) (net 5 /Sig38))
  (pad 3 thru_hole oval (at 0 5.08) (size 2.4 1.6) (drill 0.8) (layers *.Cu *.Mask) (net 36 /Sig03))
  (pad 22 thru_hole oval (at 25.4 45.72) (size 2.4 1.6) (drill 0.8) (layers *.Cu *.Mask) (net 3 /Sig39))
  (pad 2 thru_hole oval (at 0 2.54) (size 2.4 1.6) (drill 0.8) (layers *.Cu *.Mask) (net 38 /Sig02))
  (pad 21 thru_hole oval (at 25.4 48.26) (size 2.4 1.6) (drill 0.8) (layers *.Cu *.Mask) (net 1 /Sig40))
  (pad 1 thru_hole rect (at 0 0) (size 2.4 1.6) (drill 0.8) (layers *.Cu *.Mask) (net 40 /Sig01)))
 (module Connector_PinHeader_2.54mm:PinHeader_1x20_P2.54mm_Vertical (layer F.Cu) (at 151.638 77.724)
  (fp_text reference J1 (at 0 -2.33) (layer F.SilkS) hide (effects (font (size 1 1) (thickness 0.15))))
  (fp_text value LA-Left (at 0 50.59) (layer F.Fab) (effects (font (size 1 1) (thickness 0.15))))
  (pad 20 thru_hole oval (at 0 48.26) (size 1.7 1.7) (drill 1) (layers *.Cu *.Mask) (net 2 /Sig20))
  (pad 19 thru_hole oval (at 0 45.72) (size 1.7 1.7) (drill 1) (layers *.Cu *.Mask) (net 4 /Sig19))
  (pad 18 thru_hole oval (at 0 43.18) (size 1.7 1.7) (drill 1) (layers *.Cu *.Mask) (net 6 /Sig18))
  (pad 17 thru_hole oval (at 0 40.64) (size 1.7 1.7) (drill 1) (layers *.Cu *.Mask) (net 8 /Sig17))
  (pad 16 thru_hole oval (at 0 38.1) (size 1.7 1.7) (drill 1) (layers *.Cu *.Mask) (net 10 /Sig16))
  (pad 15 thru_hole oval (at 0 35.56) (size 1.7 1.7) (drill 1) (layers *.Cu *.Mask) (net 12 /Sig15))
  (pad 14 thru_hole oval (at 0 33.02) (size 1.7 1.7) (drill 1) (layers *.Cu *.Mask) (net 14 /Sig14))
  (pad 13 thru_hole oval (at 0 30.48) (size 1.7 1.7) (drill 1) (layers *.Cu *.Mask) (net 16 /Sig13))
  (pad 12 thru_hole oval (at 0 27.94) (size 1.7 1.7) (drill 1) (layers *.Cu *.Mask) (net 18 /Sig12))
  (pad 11 thru_hole oval (at 0 25.4) (size 1.7 1.7) (drill 1) (layers *.Cu *.Mask) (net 20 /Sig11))
  (pad 10 thru_hole oval (at 0 22.86) (size 1.7 1.7) (drill 1) (layers *.Cu *.Mask) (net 22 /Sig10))
  (pad 9 thru_hole oval (at 0 20.32) (size 1.7 1.7) (drill 1) (layers *.Cu *.Mask) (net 24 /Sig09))
  (pad 8 thru_hole oval (at 0 17.78) (size 1.7 1.7) (drill 1) (layers *.Cu *.Mask) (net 26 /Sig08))
  (pad 7 thru_hole oval (at 0 15.24) (size 1.7 1.7) (drill 1) (layers *.Cu *.Mask) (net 28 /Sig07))
  (pad 6 thru_hole oval (at 0 12.7) (size 1.7 1.7) (drill 1) (layers *.Cu *.Mask) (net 30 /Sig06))
  (pad 5 thru_hole oval (at 0 10.16) (size 1.7 1.7) (drill 1) (layers *.Cu *.Mask) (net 32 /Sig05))
  (pad 4 thru_hole oval (at 0 7.62) (size 1.7 1.7) (drill 1) (layers *.Cu *.Mask) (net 34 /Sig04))
  (pad 3 thru_hole oval (at 0 5.08) (size 1.7 1.7) (drill 1) (layers *.Cu *.Mask) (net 36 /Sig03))
  (pad 2 thru_hole oval (at 0 2.54) (size 1.7 1.7) (drill 1) (layers *.Cu *.Mask) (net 38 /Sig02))
  (pad 1 thru_hole rect (at 0 0) (size 1.7 1.7) (drill 1) (layers *.Cu *.Mask) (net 40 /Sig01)))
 (gr_line (start 146.558 127.508) (end 146.558 75.946) (layer Edge.Cuts) (width 0.1))
 (gr_line (start 175.26 127.508) (end 146.558 127.508) (layer Edge.Cuts) (width 0.1))
 (gr_line (start 175.26 75.946) (end 175.26 127.508) (layer Edge.Cuts) (width 0.1))
 (gr_line (start 146.558 75.946) (end 175.26 75.946) (layer Edge.Cuts) (width 0.1))
 (segment (start 148.2284 125.8824) (end 159.6136 125.8824) (width 0.3048) (layer F.Cu) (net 2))
 (segment (start 148.2284 123.3424) (end 159.6644 123.3424) (width 0.3048) (layer F.Cu) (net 4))
 (segment (start 159.6384 120.8274) (end 148.4126 120.8274) (width 0.3048) (layer F.Cu) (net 6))
 (segment (start 159.6384 118.2874) (end 148.5134 118.2874) (width 0.3048) (layer F.Cu) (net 8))
 (segment (start 159.6384 115.7474) (end 148.4126 115.7474) (width 0.3048) (layer F.Cu) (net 10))
 (segment (start 159.6384 113.2074) (end 148.4126 113.2074) (width 0.3048) (layer F.Cu) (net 12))
 (segment (start 159.6384 110.6674) (end 148.5134 110.6674) (width 0.3048) (layer F.Cu) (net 14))
 (segment (start 159.6384 108.1274) (end 148.4126 108.1274) (width 0.3048) (layer F.Cu) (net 16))
 (segment (start 159.6384 105.5874) (end 148.4126 105.5874) (width 0.3048) (layer F.Cu) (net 18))
 (segment (start 159.6384 103.0474) (end 148.5134 103.0474) (width 0.3048) (layer F.Cu) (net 20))
 (segment (start 159.6384 100.5074) (end 148.4126 100.5074) (width 0.3048) (layer F.Cu) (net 22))
 (segment (start 159.6384 97.9674) (end 148.4126 97.9674) (width 0.3048) (layer F.Cu) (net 24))
 (segment (start 159.6384 95.4274) (end 148.5134 95.4274) (width 0.3048) (layer F.Cu) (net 26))
 (segment (start 159.6384 92.8874) (end 148.4126 92.8874) (width 0.3048) (layer F.Cu) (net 28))
 (segment (start 159.6384 90.3474) (end 148.4126 90.3474) (width 0.3048) (layer F.Cu) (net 30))
 (segment (start 159.6384 87.8074) (end 148.5134 87.8074) (width 0.3048) (layer F.Cu) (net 32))
 (segment (start 159.6384 85.2674) (end 148.4126 85.2674) (width 0.3048) (layer F.Cu) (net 34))
 (segment (start 159.6384 82.7274) (end 148.4126 82.7274) (width 0.3048) (layer F.Cu) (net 36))
 (segment (start 159.6384 80.1874) (end 148.5134 80.1874) (width 0.3048) (layer F.Cu) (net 38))
 (segment (start 148.5134 80.1874) (end 148.336 80.01) (width 0.3048) (layer F.Cu) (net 38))
 (segment (start 159.6384 77.6474) (end 148.4126 77.6474) (width 0.3048) (layer F.Cu) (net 40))
 (segment (start 148.4126 77.6474) (end 148.336 77.724) (width 0.3048) (layer F.Cu) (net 40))
 (segment (start 173.6084 125.9074) (end 162.3826 125.9074) (width 0.3048) (layer F.Cu) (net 1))
 (segment (start 173.6084 123.3674) (end 162.4834 123.3674) (width 0.3048) (layer F.Cu) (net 3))
 (segment (start 173.6084 120.8274) (end 162.3826 120.8274) (width 0.3048) (layer F.Cu) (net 5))
 (segment (start 173.6084 118.2874) (end 162.3826 118.2874) (width 0.3048) (layer F.Cu) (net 7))
 (segment (start 173.6084 115.7474) (end 162.4834 115.7474) (width 0.3048) (layer F.Cu) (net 9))
 (segment (start 173.6084 113.2074) (end 162.3826 113.2074) (width 0.3048) (layer F.Cu) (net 11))
 (segment (start 173.6084 110.6674) (end 162.3826 110.6674) (width 0.3048) (layer F.Cu) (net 13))
 (segment (start 173.6084 108.1274) (end 162.4834 108.1274) (width 0.3048) (layer F.Cu) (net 15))
 (segment (start 173.6084 105.5874) (end 162.3826 105.5874) (width 0.3048) (layer F.Cu) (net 17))
 (segment (start 173.6084 103.0474) (end 162.3826 103.0474) (width 0.3048) (layer F.Cu) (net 19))
 (segment (start 173.6084 100.5074) (end 162.4834 100.5074) (width 0.3048) (layer F.Cu) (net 21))
 (segment (start 173.6084 97.9674) (end 162.3826 97.9674) (width 0.3048) (layer F.Cu) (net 23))
 (segment (start 173.6084 95.4274) (end 162.3826 95.4274) (width 0.3048) (layer F.Cu) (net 25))
 (segment (start 173.6084 92.8874) (end 162.4834 92.8874) (width 0.3048) (layer F.Cu) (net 27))
 (segment (start 173.6084 90.3474) (end 162.3826 90.3474) (width 0.3048) (layer F.Cu) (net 29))
 (segment (start 173.6084 87.8074) (end 162.3826 87.8074) (width 0.3048) (layer F.Cu) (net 31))
 (segment (start 173.6084 85.2674) (end 162.4834 85.2674) (width 0.3048) (layer F.Cu) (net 33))
 (segment (start 173.6084 82.7274) (end 162.3826 82.7274) (width 0.3048) (layer F.Cu) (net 35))
 (segment (start 162.1784 80.1874) (end 173.6594 80.1874) (width 0.3048) (layer F.Cu) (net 37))
 (segment (start 162.1784 77.6474) (end 173.4054 77.6474) (width 0.3048) (layer F.Cu) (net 39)))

